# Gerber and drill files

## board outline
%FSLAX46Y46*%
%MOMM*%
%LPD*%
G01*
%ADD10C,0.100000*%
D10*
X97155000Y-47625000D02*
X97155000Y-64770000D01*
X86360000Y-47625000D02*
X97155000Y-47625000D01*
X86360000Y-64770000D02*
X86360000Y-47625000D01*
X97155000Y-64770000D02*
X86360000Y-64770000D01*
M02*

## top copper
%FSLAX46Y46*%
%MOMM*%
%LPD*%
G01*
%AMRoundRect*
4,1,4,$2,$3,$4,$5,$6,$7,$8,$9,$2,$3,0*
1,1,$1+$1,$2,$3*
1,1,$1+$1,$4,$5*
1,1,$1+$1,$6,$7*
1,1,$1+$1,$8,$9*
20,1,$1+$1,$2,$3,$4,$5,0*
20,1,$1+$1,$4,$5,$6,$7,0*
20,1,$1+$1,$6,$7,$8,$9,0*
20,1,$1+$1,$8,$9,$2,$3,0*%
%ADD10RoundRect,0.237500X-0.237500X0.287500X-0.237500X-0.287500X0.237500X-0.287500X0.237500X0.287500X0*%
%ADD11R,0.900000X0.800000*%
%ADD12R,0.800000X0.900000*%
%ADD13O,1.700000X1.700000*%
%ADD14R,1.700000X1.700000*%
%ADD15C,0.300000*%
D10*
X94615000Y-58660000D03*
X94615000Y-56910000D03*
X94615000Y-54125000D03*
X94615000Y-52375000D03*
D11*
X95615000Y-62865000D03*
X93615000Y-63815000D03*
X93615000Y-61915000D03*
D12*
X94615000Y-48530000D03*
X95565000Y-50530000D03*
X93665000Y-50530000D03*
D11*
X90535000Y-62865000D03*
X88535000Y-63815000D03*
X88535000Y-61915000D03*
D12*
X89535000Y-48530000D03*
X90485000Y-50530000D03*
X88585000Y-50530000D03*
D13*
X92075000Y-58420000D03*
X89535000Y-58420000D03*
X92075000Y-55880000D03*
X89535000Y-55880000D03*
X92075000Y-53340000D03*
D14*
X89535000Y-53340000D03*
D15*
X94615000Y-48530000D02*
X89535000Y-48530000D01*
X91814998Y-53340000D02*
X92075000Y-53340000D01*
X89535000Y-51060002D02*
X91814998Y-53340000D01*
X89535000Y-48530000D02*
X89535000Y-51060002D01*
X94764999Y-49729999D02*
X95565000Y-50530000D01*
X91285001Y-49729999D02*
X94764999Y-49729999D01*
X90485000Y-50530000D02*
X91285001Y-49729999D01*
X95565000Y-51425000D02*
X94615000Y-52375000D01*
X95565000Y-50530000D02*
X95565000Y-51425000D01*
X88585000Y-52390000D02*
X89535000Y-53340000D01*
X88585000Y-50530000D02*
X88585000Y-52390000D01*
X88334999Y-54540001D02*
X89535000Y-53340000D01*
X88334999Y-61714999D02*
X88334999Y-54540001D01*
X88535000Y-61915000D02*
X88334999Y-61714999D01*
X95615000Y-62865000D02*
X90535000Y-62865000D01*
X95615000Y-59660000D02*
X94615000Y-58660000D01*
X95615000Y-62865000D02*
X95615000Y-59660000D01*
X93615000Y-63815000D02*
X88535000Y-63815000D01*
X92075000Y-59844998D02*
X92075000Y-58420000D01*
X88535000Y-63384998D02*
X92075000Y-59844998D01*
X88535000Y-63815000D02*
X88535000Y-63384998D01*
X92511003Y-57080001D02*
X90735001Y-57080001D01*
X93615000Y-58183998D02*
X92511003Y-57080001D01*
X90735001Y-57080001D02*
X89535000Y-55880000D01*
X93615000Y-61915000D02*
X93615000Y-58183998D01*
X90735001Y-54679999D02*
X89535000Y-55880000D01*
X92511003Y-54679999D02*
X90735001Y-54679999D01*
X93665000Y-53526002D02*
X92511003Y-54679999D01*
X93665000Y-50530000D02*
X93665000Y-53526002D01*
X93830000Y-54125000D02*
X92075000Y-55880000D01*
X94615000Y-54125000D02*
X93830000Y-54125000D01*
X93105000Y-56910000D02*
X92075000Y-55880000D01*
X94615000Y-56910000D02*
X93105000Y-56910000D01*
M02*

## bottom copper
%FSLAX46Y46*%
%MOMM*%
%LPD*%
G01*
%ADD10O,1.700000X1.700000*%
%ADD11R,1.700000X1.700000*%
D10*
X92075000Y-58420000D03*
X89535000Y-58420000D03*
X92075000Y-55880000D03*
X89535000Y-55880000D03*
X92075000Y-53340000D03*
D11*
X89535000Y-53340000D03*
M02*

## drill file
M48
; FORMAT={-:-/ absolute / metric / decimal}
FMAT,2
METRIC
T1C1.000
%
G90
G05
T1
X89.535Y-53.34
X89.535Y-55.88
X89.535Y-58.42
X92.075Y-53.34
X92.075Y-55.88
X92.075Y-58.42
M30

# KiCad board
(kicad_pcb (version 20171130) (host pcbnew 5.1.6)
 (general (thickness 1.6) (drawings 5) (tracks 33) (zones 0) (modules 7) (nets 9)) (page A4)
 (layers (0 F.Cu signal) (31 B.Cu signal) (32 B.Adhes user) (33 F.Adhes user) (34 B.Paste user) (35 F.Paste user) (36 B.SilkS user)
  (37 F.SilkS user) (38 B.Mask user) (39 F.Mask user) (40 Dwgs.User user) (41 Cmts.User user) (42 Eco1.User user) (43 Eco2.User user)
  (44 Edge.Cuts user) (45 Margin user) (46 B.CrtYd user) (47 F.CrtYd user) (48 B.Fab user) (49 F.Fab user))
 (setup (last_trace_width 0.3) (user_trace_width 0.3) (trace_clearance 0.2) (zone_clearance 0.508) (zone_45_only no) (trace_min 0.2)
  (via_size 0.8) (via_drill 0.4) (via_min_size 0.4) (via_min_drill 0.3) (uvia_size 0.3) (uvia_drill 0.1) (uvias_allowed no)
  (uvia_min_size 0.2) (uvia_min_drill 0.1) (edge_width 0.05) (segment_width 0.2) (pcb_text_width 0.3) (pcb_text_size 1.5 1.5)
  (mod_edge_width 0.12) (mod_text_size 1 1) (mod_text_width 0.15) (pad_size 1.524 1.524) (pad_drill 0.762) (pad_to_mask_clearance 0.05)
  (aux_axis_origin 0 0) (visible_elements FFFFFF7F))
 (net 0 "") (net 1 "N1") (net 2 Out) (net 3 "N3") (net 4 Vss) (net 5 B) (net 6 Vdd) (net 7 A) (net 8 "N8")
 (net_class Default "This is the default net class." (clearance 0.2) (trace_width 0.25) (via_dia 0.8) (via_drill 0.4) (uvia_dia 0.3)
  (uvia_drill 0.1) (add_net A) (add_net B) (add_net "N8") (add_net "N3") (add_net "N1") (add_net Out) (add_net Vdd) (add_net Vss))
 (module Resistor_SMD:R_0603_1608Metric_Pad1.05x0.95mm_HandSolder (layer F.Cu) (at 94.615 57.785 270)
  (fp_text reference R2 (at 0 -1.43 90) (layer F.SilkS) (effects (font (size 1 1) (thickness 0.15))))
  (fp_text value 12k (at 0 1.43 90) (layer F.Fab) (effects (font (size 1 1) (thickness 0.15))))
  (pad 2 smd roundrect (at 0.875 0 270) (size 1.05 0.95) (layers F.Cu F.Paste F.Mask) (roundrect_rratio 0.25) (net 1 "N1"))
  (pad 1 smd roundrect (at -0.875 0 270) (size 1.05 0.95) (layers F.Cu F.Paste F.Mask) (roundrect_rratio 0.25) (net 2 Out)))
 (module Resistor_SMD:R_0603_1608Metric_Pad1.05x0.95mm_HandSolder (layer F.Cu) (at 94.615 53.25 270)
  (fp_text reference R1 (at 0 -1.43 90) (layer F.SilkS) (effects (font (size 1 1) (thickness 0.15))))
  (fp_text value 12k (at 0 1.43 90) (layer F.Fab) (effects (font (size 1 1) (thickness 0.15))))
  (pad 2 smd roundrect (at 0.875 0 270) (size 1.05 0.95) (layers F.Cu F.Paste F.Mask) (roundrect_rratio 0.25) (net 2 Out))
  (pad 1 smd roundrect (at -0.875 0 270) (size 1.05 0.95) (layers F.Cu F.Paste F.Mask) (roundrect_rratio 0.25) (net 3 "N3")))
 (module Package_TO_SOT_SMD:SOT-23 (layer F.Cu) (at 94.615 62.865)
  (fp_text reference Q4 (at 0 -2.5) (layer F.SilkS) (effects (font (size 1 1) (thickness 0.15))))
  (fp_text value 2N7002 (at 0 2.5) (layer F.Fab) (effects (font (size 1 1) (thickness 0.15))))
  (pad 3 smd rect (at 1 0) (size 0.9 0.8) (layers F.Cu F.Paste F.Mask) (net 1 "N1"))
  (pad 2 smd rect (at -1 0.95) (size 0.9 0.8) (layers F.Cu F.Paste F.Mask) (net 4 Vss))
  (pad 1 smd rect (at -1 -0.95) (size 0.9 0.8) (layers F.Cu F.Paste F.Mask) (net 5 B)))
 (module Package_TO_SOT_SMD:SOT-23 (layer F.Cu) (at 94.615 49.53 90)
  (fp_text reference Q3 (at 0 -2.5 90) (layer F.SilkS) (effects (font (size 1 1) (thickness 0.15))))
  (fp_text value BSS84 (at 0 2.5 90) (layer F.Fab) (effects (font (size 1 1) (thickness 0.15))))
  (pad 3 smd rect (at 1 0 90) (size 0.9 0.8) (layers F.Cu F.Paste F.Mask) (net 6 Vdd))
  (pad 2 smd rect (at -1 0.95 90) (size 0.9 0.8) (layers F.Cu F.Paste F.Mask) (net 3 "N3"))
  (pad 1 smd rect (at -1 -0.95 90) (size 0.9 0.8) (layers F.Cu F.Paste F.Mask) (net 5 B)))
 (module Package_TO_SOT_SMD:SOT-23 (layer F.Cu) (at 89.535 62.865)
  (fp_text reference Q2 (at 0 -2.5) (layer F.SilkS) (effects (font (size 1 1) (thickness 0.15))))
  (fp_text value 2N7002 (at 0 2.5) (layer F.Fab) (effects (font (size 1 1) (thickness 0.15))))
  (pad 3 smd rect (at 1 0) (size 0.9 0.8) (layers F.Cu F.Paste F.Mask) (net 1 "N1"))
  (pad 2 smd rect (at -1 0.95) (size 0.9 0.8) (layers F.Cu F.Paste F.Mask) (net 4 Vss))
  (pad 1 smd rect (at -1 -0.95) (size 0.9 0.8) (layers F.Cu F.Paste F.Mask) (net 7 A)))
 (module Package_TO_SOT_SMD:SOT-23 (layer F.Cu) (at 89.535 49.53 90)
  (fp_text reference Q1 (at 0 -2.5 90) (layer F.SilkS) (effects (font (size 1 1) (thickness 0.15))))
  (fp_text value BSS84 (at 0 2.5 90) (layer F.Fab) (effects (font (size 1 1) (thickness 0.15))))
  (pad 3 smd rect (at 1 0 90) (size 0.9 0.8) (layers F.Cu F.Paste F.Mask) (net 6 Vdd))
  (pad 2 smd rect (at -1 0.95 90) (size 0.9 0.8) (layers F.Cu F.Paste F.Mask) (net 3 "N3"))
  (pad 1 smd rect (at -1 -0.95 90) (size 0.9 0.8) (layers F.Cu F.Paste F.Mask) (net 7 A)))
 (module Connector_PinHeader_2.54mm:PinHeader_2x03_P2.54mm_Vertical (layer F.Cu) (at 89.535 53.34)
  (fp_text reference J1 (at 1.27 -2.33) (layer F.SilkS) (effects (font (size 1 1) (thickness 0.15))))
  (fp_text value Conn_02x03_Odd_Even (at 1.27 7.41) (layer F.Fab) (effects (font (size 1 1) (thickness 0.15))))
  (pad 6 thru_hole oval (at 2.54 5.08) (size 1.7 1.7) (drill 1) (layers *.Cu *.Mask) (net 4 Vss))
  (pad 5 thru_hole oval (at 0 5.08) (size 1.7 1.7) (drill 1) (layers *.Cu *.Mask) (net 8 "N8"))
  (pad 4 thru_hole oval (at 2.54 2.54) (size 1.7 1.7) (drill 1) (layers *.Cu *.Mask) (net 2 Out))
  (pad 3 thru_hole oval (at 0 2.54) (size 1.7 1.7) (drill 1) (layers *.Cu *.Mask) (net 5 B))
  (pad 2 thru_hole oval (at 2.54 0) (size 1.7 1.7) (drill 1) (layers *.Cu *.Mask) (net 6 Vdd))
  (pad 1 thru_hole rect (at 0 0) (size 1.7 1.7) (drill 1) (layers *.Cu *.Mask) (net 7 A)))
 (gr_line (start 97.155 47.625) (end 97.155 64.77) (layer Edge.Cuts) (width 0.1))
 (gr_line (start 86.36 47.625) (end 97.155 47.625) (layer Edge.Cuts) (width 0.1))
 (gr_line (start 86.36 64.77) (end 86.36 47.625) (layer Edge.Cuts) (width 0.1))
 (gr_line (start 97.155 64.77) (end 86.36 64.77) (layer Edge.Cuts) (width 0.1))
 (segment (start 94.615 48.53) (end 89.535 48.53) (width 0.3) (layer F.Cu) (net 6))
 (segment (start 91.814998 53.34) (end 92.075 53.34) (width 0.3) (layer F.Cu) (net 6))
 (segment (start 89.535 51.060002) (end 91.814998 53.34) (width 0.3) (layer F.Cu) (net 6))
 (segment (start 89.535 48.53) (end 89.535 51.060002) (width 0.3) (layer F.Cu) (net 6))
 (segment (start 94.764999 49.729999) (end 95.565 50.53) (width 0.3) (layer F.Cu) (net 3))
 (segment (start 91.285001 49.729999) (end 94.764999 49.729999) (width 0.3) (layer F.Cu) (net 3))
 (segment (start 90.485 50.53) (end 91.285001 49.729999) (width 0.3) (layer F.Cu) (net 3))
 (segment (start 95.565 51.425) (end 94.615 52.375) (width 0.3) (layer F.Cu) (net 3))
 (segment (start 95.565 50.53) (end 95.565 51.425) (width 0.3) (layer F.Cu) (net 3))
 (segment (start 88.585 52.39) (end 89.535 53.34) (width 0.3) (layer F.Cu) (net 7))
 (segment (start 88.585 50.53) (end 88.585 52.39) (width 0.3) (layer F.Cu) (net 7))
 (segment (start 88.334999 54.540001) (end 89.535 53.34) (width 0.3) (layer F.Cu) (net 7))
 (segment (start 88.334999 61.714999) (end 88.334999 54.540001) (width 0.3) (layer F.Cu) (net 7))
 (segment (start 88.535 61.915) (end 88.334999 61.714999) (width 0.3) (layer F.Cu) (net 7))
 (segment (start 95.615 62.865) (end 90.535 62.865) (width 0.3) (layer F.Cu) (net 1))
 (segment (start 95.615 59.66) (end 94.615 58.66) (width 0.3) (layer F.Cu) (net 1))
 (segment (start 95.615 62.865) (end 95.615 59.66) (width 0.3) (layer F.Cu) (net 1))
 (segment (start 93.615 63.815) (end 88.535 63.815) (width 0.3) (layer F.Cu) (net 4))
 (segment (start 92.075 59.844998) (end 92.075 58.42) (width 0.3) (layer F.Cu) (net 4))
 (segment (start 88.535 63.384998) (end 92.075 59.844998) (width 0.3) (layer F.Cu) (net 4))
 (segment (start 88.535 63.815) (end 88.535 63.384998) (width 0.3) (layer F.Cu) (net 4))
 (segment (start 92.511003 57.080001) (end 90.735001 57.080001) (width 0.3) (layer F.Cu) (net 5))
 (segment (start 93.615 58.183998) (end 92.511003 57.080001) (width 0.3) (layer F.Cu) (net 5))
 (segment (start 90.735001 57.080001) (end 89.535 55.88) (width 0.3) (layer F.Cu) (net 5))
 (segment (start 93.615 61.915) (end 93.615 58.183998) (width 0.3) (layer F.Cu) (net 5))
 (segment (start 90.735001 54.679999) (end 89.535 55.88) (width 0.3) (layer F.Cu) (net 5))
 (segment (start 92.511003 54.679999) (end 90.735001 54.679999) (width 0.3) (layer F.Cu) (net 5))
 (segment (start 93.665 53.526002) (end 92.511003 54.679999) (width 0.3) (layer F.Cu) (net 5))
 (segment (start 93.665 50.53) (end 93.665 53.526002) (width 0.3) (layer F.Cu) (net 5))
 (segment (start 93.83 54.125) (end 92.075 55.88) (width 0.3) (layer F.Cu) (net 2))
 (segment (start 94.615 54.125) (end 93.83 54.125) (width 0.3) (layer F.Cu) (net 2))
 (segment (start 93.105 56.91) (end 92.075 55.88) (width 0.3) (layer F.Cu) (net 2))
 (segment (start 94.615 56.91) (end 93.105 56.91) (width 0.3) (layer F.Cu) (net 2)))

